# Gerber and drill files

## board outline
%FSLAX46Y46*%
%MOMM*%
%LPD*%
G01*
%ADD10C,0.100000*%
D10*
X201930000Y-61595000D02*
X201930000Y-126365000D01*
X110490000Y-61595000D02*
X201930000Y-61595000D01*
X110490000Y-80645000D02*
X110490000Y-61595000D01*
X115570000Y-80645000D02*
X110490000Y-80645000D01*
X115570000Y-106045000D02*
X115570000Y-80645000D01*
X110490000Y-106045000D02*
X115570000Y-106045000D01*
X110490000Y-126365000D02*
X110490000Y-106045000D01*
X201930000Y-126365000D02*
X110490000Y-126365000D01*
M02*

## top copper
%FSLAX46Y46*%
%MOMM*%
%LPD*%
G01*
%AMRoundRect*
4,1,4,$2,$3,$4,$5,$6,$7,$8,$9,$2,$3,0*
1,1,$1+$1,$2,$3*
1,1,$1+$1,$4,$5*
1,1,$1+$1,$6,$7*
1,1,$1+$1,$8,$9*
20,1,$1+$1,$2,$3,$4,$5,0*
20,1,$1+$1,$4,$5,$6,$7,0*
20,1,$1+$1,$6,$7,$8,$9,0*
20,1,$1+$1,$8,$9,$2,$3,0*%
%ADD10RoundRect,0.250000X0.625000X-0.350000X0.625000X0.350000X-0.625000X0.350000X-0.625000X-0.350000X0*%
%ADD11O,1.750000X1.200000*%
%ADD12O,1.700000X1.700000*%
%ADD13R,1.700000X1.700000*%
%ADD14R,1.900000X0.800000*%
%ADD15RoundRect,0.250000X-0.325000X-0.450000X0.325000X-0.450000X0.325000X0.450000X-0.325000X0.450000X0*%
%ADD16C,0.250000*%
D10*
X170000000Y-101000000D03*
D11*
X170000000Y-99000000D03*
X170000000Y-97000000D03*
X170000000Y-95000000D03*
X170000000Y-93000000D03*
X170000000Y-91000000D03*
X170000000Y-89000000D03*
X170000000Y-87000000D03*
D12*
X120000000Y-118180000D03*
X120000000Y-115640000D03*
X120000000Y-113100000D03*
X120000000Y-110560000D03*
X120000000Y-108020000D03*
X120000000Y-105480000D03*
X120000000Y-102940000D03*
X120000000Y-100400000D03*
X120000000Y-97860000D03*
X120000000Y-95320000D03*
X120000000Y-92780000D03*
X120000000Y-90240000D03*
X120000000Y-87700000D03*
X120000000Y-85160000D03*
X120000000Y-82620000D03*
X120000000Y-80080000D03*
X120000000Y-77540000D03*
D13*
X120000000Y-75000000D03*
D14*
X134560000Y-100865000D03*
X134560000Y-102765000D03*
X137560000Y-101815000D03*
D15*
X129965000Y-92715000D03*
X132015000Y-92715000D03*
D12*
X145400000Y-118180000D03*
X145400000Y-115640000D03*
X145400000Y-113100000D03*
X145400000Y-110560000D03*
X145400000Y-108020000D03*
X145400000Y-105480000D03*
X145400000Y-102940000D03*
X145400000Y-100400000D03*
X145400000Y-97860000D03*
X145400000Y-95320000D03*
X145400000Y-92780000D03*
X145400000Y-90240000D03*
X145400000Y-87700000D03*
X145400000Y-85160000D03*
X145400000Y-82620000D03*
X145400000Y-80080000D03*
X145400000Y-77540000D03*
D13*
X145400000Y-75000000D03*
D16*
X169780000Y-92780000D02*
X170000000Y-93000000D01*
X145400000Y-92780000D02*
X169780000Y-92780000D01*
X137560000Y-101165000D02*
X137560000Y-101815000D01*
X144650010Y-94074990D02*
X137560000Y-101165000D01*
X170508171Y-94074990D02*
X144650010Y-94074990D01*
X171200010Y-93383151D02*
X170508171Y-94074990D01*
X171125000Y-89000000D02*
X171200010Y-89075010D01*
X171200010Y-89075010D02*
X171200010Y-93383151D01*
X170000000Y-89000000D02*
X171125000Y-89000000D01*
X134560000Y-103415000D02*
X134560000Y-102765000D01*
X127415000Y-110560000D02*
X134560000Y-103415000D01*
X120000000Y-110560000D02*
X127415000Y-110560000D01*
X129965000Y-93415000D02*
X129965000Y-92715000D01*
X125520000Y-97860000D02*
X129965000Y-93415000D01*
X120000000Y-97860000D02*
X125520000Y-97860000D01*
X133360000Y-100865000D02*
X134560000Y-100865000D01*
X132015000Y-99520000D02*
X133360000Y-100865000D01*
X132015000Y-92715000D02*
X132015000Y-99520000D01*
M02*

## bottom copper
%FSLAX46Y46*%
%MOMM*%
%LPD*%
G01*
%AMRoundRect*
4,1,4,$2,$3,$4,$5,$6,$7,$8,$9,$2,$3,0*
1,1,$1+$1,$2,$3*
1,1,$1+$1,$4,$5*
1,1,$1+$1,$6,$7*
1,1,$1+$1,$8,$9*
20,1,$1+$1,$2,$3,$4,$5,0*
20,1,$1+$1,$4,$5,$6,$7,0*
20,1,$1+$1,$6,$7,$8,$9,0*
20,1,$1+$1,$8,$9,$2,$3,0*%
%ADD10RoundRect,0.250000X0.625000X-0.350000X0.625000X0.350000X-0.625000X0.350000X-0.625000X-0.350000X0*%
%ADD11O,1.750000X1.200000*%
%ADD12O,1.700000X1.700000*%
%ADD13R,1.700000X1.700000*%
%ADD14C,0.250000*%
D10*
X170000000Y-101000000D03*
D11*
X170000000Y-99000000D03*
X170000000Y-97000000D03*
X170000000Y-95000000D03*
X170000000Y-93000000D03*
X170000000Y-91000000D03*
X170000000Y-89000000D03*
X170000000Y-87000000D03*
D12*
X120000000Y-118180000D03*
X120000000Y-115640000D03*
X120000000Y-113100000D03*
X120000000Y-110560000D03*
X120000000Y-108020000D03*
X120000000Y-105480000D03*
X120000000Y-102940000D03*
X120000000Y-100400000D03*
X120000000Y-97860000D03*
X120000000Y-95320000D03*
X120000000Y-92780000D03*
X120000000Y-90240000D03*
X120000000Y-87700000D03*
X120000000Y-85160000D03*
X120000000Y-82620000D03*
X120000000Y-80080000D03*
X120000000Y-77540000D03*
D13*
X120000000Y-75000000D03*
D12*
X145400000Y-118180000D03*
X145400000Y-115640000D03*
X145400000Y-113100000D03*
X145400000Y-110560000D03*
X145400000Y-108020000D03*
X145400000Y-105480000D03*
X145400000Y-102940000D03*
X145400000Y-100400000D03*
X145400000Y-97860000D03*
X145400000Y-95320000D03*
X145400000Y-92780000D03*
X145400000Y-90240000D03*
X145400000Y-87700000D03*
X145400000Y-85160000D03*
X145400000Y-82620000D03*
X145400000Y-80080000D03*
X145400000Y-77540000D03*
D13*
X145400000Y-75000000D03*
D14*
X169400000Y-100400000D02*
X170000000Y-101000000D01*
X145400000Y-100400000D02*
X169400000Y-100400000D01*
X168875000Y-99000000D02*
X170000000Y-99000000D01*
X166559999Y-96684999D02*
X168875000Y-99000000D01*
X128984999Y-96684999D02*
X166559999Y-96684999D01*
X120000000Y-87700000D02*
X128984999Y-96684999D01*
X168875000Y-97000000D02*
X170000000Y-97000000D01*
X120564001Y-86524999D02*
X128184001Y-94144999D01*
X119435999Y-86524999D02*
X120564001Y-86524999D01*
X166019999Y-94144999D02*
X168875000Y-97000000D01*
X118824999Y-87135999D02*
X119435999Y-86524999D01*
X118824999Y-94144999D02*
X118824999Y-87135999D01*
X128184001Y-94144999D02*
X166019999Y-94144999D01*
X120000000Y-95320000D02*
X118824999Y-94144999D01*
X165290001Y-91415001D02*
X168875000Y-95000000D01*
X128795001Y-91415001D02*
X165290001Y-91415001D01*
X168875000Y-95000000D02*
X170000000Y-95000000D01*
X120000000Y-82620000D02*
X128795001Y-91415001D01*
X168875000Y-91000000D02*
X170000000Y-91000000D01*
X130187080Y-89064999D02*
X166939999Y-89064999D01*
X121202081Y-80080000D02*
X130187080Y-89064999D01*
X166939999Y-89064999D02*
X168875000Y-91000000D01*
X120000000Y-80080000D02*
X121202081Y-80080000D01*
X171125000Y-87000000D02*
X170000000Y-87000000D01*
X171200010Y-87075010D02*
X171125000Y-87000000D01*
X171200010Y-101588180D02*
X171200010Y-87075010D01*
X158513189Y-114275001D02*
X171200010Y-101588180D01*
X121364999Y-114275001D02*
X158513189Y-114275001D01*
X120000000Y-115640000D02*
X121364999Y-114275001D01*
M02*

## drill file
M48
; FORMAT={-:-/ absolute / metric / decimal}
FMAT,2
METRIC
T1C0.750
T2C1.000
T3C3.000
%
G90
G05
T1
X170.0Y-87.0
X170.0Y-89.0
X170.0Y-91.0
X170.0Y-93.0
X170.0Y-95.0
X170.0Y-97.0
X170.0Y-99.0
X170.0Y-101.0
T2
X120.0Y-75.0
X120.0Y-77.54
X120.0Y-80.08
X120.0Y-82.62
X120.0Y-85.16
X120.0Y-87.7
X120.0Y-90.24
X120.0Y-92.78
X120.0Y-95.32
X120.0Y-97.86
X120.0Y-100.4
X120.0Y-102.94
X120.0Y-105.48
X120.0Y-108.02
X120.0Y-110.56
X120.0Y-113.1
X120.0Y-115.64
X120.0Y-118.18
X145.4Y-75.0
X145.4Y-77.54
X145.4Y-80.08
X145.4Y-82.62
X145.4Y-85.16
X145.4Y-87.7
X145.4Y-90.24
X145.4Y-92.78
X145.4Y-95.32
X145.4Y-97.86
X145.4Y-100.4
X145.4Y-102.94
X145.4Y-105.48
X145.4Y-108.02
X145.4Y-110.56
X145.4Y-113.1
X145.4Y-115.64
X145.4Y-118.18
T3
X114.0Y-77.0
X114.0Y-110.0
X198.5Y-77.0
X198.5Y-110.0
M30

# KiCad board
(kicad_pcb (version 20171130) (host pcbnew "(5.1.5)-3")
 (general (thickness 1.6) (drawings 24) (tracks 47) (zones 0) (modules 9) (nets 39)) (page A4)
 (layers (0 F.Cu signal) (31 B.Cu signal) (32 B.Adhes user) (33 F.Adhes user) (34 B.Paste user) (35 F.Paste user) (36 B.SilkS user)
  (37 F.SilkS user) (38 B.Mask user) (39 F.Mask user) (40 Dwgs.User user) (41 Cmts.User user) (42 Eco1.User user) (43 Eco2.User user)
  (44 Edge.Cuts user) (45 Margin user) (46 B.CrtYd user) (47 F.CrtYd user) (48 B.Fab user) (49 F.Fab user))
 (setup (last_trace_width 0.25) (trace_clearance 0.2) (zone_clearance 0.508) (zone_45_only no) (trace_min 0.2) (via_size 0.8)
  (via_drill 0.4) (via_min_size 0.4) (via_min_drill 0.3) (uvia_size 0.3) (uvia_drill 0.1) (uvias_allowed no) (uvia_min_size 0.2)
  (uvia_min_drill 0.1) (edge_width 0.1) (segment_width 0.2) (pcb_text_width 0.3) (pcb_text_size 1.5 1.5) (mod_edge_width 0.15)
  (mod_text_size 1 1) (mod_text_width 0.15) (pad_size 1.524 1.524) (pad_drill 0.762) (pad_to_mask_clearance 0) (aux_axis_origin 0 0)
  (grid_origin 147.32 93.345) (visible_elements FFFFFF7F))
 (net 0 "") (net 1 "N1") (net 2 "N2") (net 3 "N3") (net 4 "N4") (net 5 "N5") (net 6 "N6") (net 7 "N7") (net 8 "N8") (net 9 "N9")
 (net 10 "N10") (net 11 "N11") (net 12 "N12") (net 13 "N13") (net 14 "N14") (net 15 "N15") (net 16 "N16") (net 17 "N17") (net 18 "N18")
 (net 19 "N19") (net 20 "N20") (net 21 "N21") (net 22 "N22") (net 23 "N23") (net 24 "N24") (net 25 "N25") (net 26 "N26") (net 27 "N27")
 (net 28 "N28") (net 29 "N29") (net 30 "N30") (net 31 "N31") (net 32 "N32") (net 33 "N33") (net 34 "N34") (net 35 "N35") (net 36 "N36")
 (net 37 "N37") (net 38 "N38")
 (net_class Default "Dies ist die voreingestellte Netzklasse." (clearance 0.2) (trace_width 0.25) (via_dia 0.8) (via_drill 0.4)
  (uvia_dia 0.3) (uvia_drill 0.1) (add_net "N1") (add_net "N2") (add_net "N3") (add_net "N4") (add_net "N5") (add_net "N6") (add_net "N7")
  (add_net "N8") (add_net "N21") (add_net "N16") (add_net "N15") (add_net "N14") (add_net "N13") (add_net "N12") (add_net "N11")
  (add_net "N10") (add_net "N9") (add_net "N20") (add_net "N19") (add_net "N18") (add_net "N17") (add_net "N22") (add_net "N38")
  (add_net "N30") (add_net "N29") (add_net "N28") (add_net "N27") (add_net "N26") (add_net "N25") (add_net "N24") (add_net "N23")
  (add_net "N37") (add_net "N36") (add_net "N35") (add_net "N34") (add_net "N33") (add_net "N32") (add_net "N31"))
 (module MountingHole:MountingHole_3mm (layer F.Cu) (at 114 77)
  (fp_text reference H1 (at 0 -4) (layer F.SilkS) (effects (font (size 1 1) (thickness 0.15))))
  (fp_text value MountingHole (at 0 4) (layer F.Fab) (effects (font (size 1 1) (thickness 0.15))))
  (pad 1 np_thru_hole circle (at 0 0) (size 3 3) (drill 3) (layers *.Cu *.Mask)))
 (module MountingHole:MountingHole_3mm (layer F.Cu) (at 198.5 110)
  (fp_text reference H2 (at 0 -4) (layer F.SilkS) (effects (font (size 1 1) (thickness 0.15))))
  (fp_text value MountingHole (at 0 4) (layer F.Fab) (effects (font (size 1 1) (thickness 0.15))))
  (pad 1 np_thru_hole circle (at 0 0) (size 3 3) (drill 3) (layers *.Cu *.Mask)))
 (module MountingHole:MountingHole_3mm (layer F.Cu) (at 198.5 77)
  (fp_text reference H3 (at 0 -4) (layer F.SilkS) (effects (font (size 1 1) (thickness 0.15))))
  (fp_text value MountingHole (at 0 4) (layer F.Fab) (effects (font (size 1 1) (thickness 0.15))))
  (pad 1 np_thru_hole circle (at 0 0) (size 3 3) (drill 3) (layers *.Cu *.Mask)))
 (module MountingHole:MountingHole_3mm (layer F.Cu) (at 114 110)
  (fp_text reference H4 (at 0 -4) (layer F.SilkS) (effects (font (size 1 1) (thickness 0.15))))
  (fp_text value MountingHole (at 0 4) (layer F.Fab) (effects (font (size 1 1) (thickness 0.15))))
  (pad 1 np_thru_hole circle (at 0 0) (size 3 3) (drill 3) (layers *.Cu *.Mask)))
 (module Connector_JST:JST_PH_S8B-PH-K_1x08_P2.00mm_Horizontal (layer B.Cu) (at 170 101 90)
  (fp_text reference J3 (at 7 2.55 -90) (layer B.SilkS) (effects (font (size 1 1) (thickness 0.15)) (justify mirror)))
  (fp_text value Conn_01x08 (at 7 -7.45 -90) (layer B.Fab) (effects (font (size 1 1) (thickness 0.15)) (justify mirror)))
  (pad 1 thru_hole roundrect (at 0 0 90) (size 1.2 1.75) (drill 0.75) (layers *.Cu *.Mask) (roundrect_rratio 0.208333) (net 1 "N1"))
  (pad 2 thru_hole oval (at 2 0 90) (size 1.2 1.75) (drill 0.75) (layers *.Cu *.Mask) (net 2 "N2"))
  (pad 3 thru_hole oval (at 4 0 90) (size 1.2 1.75) (drill 0.75) (layers *.Cu *.Mask) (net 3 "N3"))
  (pad 4 thru_hole oval (at 6 0 90) (size 1.2 1.75) (drill 0.75) (layers *.Cu *.Mask) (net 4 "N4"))
  (pad 5 thru_hole oval (at 8 0 90) (size 1.2 1.75) (drill 0.75) (layers *.Cu *.Mask) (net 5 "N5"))
  (pad 6 thru_hole oval (at 10 0 90) (size 1.2 1.75) (drill 0.75) (layers *.Cu *.Mask) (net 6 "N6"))
  (pad 7 thru_hole oval (at 12 0 90) (size 1.2 1.75) (drill 0.75) (layers *.Cu *.Mask) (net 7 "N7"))
  (pad 8 thru_hole oval (at 14 0 90) (size 1.2 1.75) (drill 0.75) (layers *.Cu *.Mask) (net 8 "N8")))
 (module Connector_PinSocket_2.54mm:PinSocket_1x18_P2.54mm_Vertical (layer F.Cu) (at 120 75)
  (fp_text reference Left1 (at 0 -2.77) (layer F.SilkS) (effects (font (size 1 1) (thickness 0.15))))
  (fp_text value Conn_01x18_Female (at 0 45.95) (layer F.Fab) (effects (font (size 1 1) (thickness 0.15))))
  (pad 18 thru_hole oval (at 0 43.18) (size 1.7 1.7) (drill 1) (layers *.Cu *.Mask) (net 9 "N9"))
  (pad 17 thru_hole oval (at 0 40.64) (size 1.7 1.7) (drill 1) (layers *.Cu *.Mask) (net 8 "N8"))
  (pad 16 thru_hole oval (at 0 38.1) (size 1.7 1.7) (drill 1) (layers *.Cu *.Mask) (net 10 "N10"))
  (pad 15 thru_hole oval (at 0 35.56) (size 1.7 1.7) (drill 1) (layers *.Cu *.Mask) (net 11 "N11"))
  (pad 14 thru_hole oval (at 0 33.02) (size 1.7 1.7) (drill 1) (layers *.Cu *.Mask) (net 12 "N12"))
  (pad 13 thru_hole oval (at 0 30.48) (size 1.7 1.7) (drill 1) (layers *.Cu *.Mask) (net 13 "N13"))
  (pad 12 thru_hole oval (at 0 27.94) (size 1.7 1.7) (drill 1) (layers *.Cu *.Mask) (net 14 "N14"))
  (pad 11 thru_hole oval (at 0 25.4) (size 1.7 1.7) (drill 1) (layers *.Cu *.Mask) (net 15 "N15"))
  (pad 10 thru_hole oval (at 0 22.86) (size 1.7 1.7) (drill 1) (layers *.Cu *.Mask) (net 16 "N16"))
  (pad 9 thru_hole oval (at 0 20.32) (size 1.7 1.7) (drill 1) (layers *.Cu *.Mask) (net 3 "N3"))
  (pad 8 thru_hole oval (at 0 17.78) (size 1.7 1.7) (drill 1) (layers *.Cu *.Mask) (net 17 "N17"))
  (pad 7 thru_hole oval (at 0 15.24) (size 1.7 1.7) (drill 1) (layers *.Cu *.Mask) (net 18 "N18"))
  (pad 6 thru_hole oval (at 0 12.7) (size 1.7 1.7) (drill 1) (layers *.Cu *.Mask) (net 2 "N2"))
  (pad 5 thru_hole oval (at 0 10.16) (size 1.7 1.7) (drill 1) (layers *.Cu *.Mask) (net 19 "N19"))
  (pad 4 thru_hole oval (at 0 7.62) (size 1.7 1.7) (drill 1) (layers *.Cu *.Mask) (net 4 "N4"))
  (pad 3 thru_hole oval (at 0 5.08) (size 1.7 1.7) (drill 1) (layers *.Cu *.Mask) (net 6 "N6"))
  (pad 2 thru_hole oval (at 0 2.54) (size 1.7 1.7) (drill 1) (layers *.Cu *.Mask) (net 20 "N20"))
  (pad 1 thru_hole rect (at 0 0) (size 1.7 1.7) (drill 1) (layers *.Cu *.Mask) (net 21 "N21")))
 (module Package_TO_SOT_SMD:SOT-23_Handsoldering (layer F.Cu) (at 136.06 101.815)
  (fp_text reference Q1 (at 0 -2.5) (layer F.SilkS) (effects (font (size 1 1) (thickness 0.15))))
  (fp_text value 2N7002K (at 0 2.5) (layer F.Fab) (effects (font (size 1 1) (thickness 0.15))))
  (pad 1 smd rect (at -1.5 -0.95) (size 1.9 0.8) (layers F.Cu F.Paste F.Mask) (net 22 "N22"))
  (pad 2 smd rect (at -1.5 0.95) (size 1.9 0.8) (layers F.Cu F.Paste F.Mask) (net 11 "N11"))
  (pad 3 smd rect (at 1.5 0) (size 1.9 0.8) (layers F.Cu F.Paste F.Mask) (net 7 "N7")))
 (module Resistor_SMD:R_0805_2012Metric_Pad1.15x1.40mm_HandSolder (layer F.Cu) (at 130.99 92.715)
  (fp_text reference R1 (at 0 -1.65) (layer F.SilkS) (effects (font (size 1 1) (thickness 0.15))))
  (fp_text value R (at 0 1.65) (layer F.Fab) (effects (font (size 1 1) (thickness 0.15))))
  (pad 1 smd roundrect (at -1.025 0) (size 1.15 1.4) (layers F.Cu F.Paste F.Mask) (roundrect_rratio 0.217391) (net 16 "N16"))
  (pad 2 smd roundrect (at 1.025 0) (size 1.15 1.4) (layers F.Cu F.Paste F.Mask) (roundrect_rratio 0.217391) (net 22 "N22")))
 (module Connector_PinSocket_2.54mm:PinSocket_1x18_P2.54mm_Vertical (layer F.Cu) (at 145.4 75)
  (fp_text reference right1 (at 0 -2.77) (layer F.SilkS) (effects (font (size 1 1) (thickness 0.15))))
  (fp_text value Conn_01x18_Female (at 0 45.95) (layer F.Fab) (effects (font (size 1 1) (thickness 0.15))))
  (pad 18 thru_hole oval (at 0 43.18) (size 1.7 1.7) (drill 1) (layers *.Cu *.Mask) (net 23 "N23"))
  (pad 17 thru_hole oval (at 0 40.64) (size 1.7 1.7) (drill 1) (layers *.Cu *.Mask) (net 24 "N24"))
  (pad 16 thru_hole oval (at 0 38.1) (size 1.7 1.7) (drill 1) (layers *.Cu *.Mask) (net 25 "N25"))
  (pad 15 thru_hole oval (at 0 35.56) (size 1.7 1.7) (drill 1) (layers *.Cu *.Mask) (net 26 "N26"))
  (pad 14 thru_hole oval (at 0 33.02) (size 1.7 1.7) (drill 1) (layers *.Cu *.Mask) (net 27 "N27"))
  (pad 13 thru_hole oval (at 0 30.48) (size 1.7 1.7) (drill 1) (layers *.Cu *.Mask) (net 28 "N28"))
  (pad 12 thru_hole oval (at 0 27.94) (size 1.7 1.7) (drill 1) (layers *.Cu *.Mask) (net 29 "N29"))
  (pad 11 thru_hole oval (at 0 25.4) (size 1.7 1.7) (drill 1) (layers *.Cu *.Mask) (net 1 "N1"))
  (pad 10 thru_hole oval (at 0 22.86) (size 1.7 1.7) (drill 1) (layers *.Cu *.Mask) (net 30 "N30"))
  (pad 9 thru_hole oval (at 0 20.32) (size 1.7 1.7) (drill 1) (layers *.Cu *.Mask) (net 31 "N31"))
  (pad 8 thru_hole oval (at 0 17.78) (size 1.7 1.7) (drill 1) (layers *.Cu *.Mask) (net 5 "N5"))
  (pad 7 thru_hole oval (at 0 15.24) (size 1.7 1.7) (drill 1) (layers *.Cu *.Mask) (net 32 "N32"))
  (pad 6 thru_hole oval (at 0 12.7) (size 1.7 1.7) (drill 1) (layers *.Cu *.Mask) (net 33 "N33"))
  (pad 5 thru_hole oval (at 0 10.16) (size 1.7 1.7) (drill 1) (layers *.Cu *.Mask) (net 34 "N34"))
  (pad 4 thru_hole oval (at 0 7.62) (size 1.7 1.7) (drill 1) (layers *.Cu *.Mask) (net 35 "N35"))
  (pad 3 thru_hole oval (at 0 5.08) (size 1.7 1.7) (drill 1) (layers *.Cu *.Mask) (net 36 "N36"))
  (pad 2 thru_hole oval (at 0 2.54) (size 1.7 1.7) (drill 1) (layers *.Cu *.Mask) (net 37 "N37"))
  (pad 1 thru_hole rect (at 0 0) (size 1.7 1.7) (drill 1) (layers *.Cu *.Mask) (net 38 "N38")))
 (gr_line (start 201.93 61.595) (end 201.93 126.365) (layer Edge.Cuts) (width 0.1))
 (gr_line (start 110.49 61.595) (end 201.93 61.595) (layer Edge.Cuts) (width 0.1))
 (gr_line (start 110.49 80.645) (end 110.49 61.595) (layer Edge.Cuts) (width 0.1))
 (gr_line (start 115.57 80.645) (end 110.49 80.645) (layer Edge.Cuts) (width 0.1))
 (gr_line (start 115.57 106.045) (end 115.57 80.645) (layer Edge.Cuts) (width 0.1))
 (gr_line (start 110.49 106.045) (end 115.57 106.045) (layer Edge.Cuts) (width 0.1))
 (gr_line (start 110.49 126.365) (end 110.49 106.045) (layer Edge.Cuts) (width 0.1))
 (gr_line (start 201.93 126.365) (end 110.49 126.365) (layer Edge.Cuts) (width 0.1))
 (segment (start 169.4 100.4) (end 170 101) (width 0.25) (layer B.Cu) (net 1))
 (segment (start 145.4 100.4) (end 169.4 100.4) (width 0.25) (layer B.Cu) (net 1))
 (segment (start 168.875 99) (end 170 99) (width 0.25) (layer B.Cu) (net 2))
 (segment (start 166.559999 96.684999) (end 168.875 99) (width 0.25) (layer B.Cu) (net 2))
 (segment (start 128.984999 96.684999) (end 166.559999 96.684999) (width 0.25) (layer B.Cu) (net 2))
 (segment (start 120 87.7) (end 128.984999 96.684999) (width 0.25) (layer B.Cu) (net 2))
 (segment (start 168.875 97) (end 170 97) (width 0.25) (layer B.Cu) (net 3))
 (segment (start 120.564001 86.524999) (end 128.184001 94.144999) (width 0.25) (layer B.Cu) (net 3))
 (segment (start 119.435999 86.524999) (end 120.564001 86.524999) (width 0.25) (layer B.Cu) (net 3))
 (segment (start 166.019999 94.144999) (end 168.875 97) (width 0.25) (layer B.Cu) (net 3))
 (segment (start 118.824999 87.135999) (end 119.435999 86.524999) (width 0.25) (layer B.Cu) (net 3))
 (segment (start 118.824999 94.144999) (end 118.824999 87.135999) (width 0.25) (layer B.Cu) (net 3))
 (segment (start 128.184001 94.144999) (end 166.019999 94.144999) (width 0.25) (layer B.Cu) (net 3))
 (segment (start 120 95.32) (end 118.824999 94.144999) (width 0.25) (layer B.Cu) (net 3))
 (segment (start 165.290001 91.415001) (end 168.875 95) (width 0.25) (layer B.Cu) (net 4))
 (segment (start 128.795001 91.415001) (end 165.290001 91.415001) (width 0.25) (layer B.Cu) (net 4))
 (segment (start 168.875 95) (end 170 95) (width 0.25) (layer B.Cu) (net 4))
 (segment (start 120 82.62) (end 128.795001 91.415001) (width 0.25) (layer B.Cu) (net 4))
 (segment (start 169.78 92.78) (end 170 93) (width 0.25) (layer F.Cu) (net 5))
 (segment (start 145.4 92.78) (end 169.78 92.78) (width 0.25) (layer F.Cu) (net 5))
 (segment (start 168.875 91) (end 170 91) (width 0.25) (layer B.Cu) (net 6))
 (segment (start 130.18708 89.064999) (end 166.939999 89.064999) (width 0.25) (layer B.Cu) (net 6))
 (segment (start 121.202081 80.08) (end 130.18708 89.064999) (width 0.25) (layer B.Cu) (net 6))
 (segment (start 166.939999 89.064999) (end 168.875 91) (width 0.25) (layer B.Cu) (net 6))
 (segment (start 120 80.08) (end 121.202081 80.08) (width 0.25) (layer B.Cu) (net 6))
 (segment (start 137.56 101.165) (end 137.56 101.815) (width 0.25) (layer F.Cu) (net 7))
 (segment (start 144.65001 94.07499) (end 137.56 101.165) (width 0.25) (layer F.Cu) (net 7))
 (segment (start 170.508171 94.07499) (end 144.65001 94.07499) (width 0.25) (layer F.Cu) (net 7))
 (segment (start 171.20001 93.383151) (end 170.508171 94.07499) (width 0.25) (layer F.Cu) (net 7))
 (segment (start 171.125 89) (end 171.20001 89.07501) (width 0.25) (layer F.Cu) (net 7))
 (segment (start 171.20001 89.07501) (end 171.20001 93.383151) (width 0.25) (layer F.Cu) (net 7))
 (segment (start 170 89) (end 171.125 89) (width 0.25) (layer F.Cu) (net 7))
 (segment (start 171.125 87) (end 170 87) (width 0.25) (layer B.Cu) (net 8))
 (segment (start 171.20001 87.07501) (end 171.125 87) (width 0.25) (layer B.Cu) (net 8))
 (segment (start 171.20001 101.58818) (end 171.20001 87.07501) (width 0.25) (layer B.Cu) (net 8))
 (segment (start 158.513189 114.275001) (end 171.20001 101.58818) (width 0.25) (layer B.Cu) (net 8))
 (segment (start 121.364999 114.275001) (end 158.513189 114.275001) (width 0.25) (layer B.Cu) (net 8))
 (segment (start 120 115.64) (end 121.364999 114.275001) (width 0.25) (layer B.Cu) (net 8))
 (segment (start 134.56 103.415) (end 134.56 102.765) (width 0.25) (layer F.Cu) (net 11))
 (segment (start 127.415 110.56) (end 134.56 103.415) (width 0.25) (layer F.Cu) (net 11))
 (segment (start 120 110.56) (end 127.415 110.56) (width 0.25) (layer F.Cu) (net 11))
 (segment (start 129.965 93.415) (end 129.965 92.715) (width 0.25) (layer F.Cu) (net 16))
 (segment (start 125.52 97.86) (end 129.965 93.415) (width 0.25) (layer F.Cu) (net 16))
 (segment (start 120 97.86) (end 125.52 97.86) (width 0.25) (layer F.Cu) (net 16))
 (segment (start 133.36 100.865) (end 134.56 100.865) (width 0.25) (layer F.Cu) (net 22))
 (segment (start 132.015 99.52) (end 133.36 100.865) (width 0.25) (layer F.Cu) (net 22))
 (segment (start 132.015 92.715) (end 132.015 99.52) (width 0.25) (layer F.Cu) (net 22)))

